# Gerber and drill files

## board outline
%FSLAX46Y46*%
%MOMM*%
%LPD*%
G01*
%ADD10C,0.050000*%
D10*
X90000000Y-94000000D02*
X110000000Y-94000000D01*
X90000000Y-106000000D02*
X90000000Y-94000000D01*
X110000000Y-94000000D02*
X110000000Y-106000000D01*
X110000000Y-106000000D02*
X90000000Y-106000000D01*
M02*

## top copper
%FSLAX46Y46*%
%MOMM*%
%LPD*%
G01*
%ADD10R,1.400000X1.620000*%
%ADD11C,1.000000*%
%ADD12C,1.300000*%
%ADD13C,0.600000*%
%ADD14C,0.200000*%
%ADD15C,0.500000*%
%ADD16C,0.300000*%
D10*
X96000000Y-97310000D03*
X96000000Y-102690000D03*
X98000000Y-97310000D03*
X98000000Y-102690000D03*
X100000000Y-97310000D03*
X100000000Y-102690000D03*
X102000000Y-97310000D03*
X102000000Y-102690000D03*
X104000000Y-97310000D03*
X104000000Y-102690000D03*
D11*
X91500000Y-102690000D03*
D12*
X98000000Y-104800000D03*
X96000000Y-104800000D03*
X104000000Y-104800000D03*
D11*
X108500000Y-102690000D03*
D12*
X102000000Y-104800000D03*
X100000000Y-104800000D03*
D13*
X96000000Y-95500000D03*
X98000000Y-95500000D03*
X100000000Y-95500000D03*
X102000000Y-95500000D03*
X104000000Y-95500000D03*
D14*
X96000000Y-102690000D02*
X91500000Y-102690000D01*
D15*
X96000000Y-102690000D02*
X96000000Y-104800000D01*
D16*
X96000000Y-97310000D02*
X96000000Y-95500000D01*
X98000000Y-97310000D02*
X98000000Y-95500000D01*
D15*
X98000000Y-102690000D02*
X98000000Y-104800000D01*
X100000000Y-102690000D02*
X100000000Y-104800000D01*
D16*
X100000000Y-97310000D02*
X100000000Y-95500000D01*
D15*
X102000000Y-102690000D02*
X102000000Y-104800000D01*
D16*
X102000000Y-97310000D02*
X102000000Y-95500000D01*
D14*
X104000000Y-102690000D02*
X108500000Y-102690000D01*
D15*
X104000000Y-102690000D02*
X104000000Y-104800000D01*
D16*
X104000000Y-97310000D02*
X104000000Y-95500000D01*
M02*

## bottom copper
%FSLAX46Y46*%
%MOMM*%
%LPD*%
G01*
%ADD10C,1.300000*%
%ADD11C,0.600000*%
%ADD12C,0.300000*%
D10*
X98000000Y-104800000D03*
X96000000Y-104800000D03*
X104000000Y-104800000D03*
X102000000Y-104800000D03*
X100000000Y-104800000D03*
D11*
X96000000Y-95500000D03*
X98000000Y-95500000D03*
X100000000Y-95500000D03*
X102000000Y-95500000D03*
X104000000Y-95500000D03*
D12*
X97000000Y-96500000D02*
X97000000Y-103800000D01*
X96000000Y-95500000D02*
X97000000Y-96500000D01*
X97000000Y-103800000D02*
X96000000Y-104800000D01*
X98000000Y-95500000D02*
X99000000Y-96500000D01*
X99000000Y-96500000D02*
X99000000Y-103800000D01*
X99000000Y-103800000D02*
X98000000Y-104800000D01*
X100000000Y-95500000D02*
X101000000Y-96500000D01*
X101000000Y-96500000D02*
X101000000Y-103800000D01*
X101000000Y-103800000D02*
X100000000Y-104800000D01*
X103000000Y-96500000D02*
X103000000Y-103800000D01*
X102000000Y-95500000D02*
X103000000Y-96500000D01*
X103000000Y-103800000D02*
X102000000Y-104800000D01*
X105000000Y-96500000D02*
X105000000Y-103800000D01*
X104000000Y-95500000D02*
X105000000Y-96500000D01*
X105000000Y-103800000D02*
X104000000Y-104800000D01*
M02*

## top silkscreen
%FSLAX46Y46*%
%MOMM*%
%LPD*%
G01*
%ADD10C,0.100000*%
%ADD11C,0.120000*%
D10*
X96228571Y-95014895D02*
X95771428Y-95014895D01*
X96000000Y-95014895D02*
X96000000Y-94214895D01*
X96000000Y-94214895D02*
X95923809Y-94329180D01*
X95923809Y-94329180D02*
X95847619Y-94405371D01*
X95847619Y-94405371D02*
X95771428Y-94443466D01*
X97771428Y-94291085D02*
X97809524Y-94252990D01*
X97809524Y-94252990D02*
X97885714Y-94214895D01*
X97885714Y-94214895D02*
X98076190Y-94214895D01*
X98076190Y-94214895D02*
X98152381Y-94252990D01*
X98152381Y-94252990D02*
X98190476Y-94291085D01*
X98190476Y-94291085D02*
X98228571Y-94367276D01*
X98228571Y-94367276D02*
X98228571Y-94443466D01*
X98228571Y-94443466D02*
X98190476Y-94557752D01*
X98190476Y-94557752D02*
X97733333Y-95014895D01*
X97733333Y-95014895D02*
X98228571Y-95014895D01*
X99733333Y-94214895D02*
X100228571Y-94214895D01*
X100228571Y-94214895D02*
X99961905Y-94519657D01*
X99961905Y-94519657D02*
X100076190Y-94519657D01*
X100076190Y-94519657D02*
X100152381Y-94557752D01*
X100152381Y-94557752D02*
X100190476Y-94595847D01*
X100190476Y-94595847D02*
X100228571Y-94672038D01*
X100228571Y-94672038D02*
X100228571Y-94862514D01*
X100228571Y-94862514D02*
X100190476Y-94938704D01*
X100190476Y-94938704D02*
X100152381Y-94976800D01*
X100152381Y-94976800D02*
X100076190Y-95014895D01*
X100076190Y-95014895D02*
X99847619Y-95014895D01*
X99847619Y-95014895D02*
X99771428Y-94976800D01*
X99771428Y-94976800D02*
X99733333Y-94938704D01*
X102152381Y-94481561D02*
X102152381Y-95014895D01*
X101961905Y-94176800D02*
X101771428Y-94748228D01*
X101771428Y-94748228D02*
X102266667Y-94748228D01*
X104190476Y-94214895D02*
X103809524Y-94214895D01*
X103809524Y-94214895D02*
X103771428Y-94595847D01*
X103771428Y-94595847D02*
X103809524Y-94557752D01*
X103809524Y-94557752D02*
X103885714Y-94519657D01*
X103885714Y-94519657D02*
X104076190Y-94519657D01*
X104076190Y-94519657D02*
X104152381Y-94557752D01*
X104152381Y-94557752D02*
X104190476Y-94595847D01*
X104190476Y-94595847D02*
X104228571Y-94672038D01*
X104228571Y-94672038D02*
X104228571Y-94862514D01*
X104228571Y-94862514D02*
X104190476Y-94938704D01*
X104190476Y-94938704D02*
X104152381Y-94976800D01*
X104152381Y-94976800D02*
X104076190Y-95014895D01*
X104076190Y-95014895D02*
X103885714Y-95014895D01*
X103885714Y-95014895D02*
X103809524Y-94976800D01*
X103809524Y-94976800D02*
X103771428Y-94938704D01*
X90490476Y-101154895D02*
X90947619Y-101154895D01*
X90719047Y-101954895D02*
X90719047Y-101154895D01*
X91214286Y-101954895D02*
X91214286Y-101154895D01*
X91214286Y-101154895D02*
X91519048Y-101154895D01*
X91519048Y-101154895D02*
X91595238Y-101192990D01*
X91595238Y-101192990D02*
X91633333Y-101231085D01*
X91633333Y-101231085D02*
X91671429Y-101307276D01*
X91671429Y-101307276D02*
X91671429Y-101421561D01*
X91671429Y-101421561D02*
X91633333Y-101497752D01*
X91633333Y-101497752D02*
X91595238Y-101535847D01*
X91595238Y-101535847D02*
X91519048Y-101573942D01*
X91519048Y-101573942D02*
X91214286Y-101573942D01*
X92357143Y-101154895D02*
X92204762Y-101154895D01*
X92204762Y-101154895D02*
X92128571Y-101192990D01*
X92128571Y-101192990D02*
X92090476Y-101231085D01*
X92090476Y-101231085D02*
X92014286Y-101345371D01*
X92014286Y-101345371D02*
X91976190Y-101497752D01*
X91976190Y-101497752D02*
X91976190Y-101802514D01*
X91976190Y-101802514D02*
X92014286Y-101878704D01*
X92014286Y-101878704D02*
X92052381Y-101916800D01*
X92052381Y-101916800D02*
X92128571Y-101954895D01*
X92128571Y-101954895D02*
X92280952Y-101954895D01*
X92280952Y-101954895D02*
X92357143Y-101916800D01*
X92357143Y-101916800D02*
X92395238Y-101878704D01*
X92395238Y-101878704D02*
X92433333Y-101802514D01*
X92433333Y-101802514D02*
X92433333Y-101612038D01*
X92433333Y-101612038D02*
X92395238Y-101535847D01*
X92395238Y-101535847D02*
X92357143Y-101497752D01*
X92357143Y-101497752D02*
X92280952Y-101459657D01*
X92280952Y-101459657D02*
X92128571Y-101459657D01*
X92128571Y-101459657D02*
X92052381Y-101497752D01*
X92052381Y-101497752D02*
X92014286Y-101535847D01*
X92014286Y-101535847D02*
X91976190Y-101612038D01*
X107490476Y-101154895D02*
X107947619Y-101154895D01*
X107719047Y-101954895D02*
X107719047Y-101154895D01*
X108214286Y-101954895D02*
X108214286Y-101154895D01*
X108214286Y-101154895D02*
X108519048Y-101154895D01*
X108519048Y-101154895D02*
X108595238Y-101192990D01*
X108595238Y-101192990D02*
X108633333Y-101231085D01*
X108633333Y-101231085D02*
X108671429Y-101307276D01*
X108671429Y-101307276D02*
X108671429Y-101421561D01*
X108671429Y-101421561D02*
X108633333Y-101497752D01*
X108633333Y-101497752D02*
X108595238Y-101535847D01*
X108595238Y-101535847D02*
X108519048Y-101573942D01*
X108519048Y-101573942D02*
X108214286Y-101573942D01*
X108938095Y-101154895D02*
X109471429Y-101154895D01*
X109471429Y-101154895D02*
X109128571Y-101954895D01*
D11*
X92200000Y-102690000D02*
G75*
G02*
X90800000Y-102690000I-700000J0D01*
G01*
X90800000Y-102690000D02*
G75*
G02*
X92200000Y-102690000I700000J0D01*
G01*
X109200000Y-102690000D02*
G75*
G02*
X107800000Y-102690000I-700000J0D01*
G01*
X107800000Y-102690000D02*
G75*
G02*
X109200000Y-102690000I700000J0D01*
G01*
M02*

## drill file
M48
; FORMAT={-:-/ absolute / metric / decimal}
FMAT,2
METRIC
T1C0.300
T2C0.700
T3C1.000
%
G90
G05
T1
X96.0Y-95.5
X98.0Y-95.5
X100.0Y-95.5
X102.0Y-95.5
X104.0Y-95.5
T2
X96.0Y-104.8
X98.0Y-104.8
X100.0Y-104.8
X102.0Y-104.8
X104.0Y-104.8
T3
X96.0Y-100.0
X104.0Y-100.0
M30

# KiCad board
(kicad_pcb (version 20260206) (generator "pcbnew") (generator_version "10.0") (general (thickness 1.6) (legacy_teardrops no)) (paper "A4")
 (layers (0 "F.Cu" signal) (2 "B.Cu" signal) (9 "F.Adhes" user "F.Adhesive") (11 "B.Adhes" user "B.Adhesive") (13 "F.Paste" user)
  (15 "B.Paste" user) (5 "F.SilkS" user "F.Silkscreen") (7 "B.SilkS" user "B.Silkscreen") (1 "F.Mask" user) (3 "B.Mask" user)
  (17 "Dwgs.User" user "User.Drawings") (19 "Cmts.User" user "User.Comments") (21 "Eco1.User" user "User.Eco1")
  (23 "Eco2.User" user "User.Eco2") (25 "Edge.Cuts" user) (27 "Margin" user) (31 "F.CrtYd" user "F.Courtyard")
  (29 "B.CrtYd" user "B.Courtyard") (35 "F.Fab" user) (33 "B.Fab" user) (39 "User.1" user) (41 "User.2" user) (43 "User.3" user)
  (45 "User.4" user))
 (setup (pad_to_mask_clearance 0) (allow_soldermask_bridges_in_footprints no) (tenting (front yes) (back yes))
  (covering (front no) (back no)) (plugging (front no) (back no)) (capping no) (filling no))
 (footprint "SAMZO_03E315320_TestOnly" (layer "F.Cu") (at 100 100)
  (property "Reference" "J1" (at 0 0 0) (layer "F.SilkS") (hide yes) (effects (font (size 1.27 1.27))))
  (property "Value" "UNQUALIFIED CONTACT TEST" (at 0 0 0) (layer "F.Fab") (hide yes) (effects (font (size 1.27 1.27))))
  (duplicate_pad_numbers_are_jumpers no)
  (pad "" np_thru_hole circle (at -4 0) (size 1 1) (drill 1) (layers "*.Cu"))
  (pad "" np_thru_hole circle (at 4 0) (size 1 1) (drill 1) (layers "*.Cu"))
  (pad "1" smd rect (at -4 -2.69) (size 1.4 1.62) (layers "F.Cu" "F.Mask" "F.Paste") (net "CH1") (thermal_bridge_angle 45))
  (pad "1" smd rect (at -4 2.69) (size 1.4 1.62) (layers "F.Cu" "F.Mask" "F.Paste") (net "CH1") (thermal_bridge_angle 45))
  (pad "2" smd rect (at -2 -2.69) (size 1.4 1.62) (layers "F.Cu" "F.Mask" "F.Paste") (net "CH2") (thermal_bridge_angle 45))
  (pad "2" smd rect (at -2 2.69) (size 1.4 1.62) (layers "F.Cu" "F.Mask" "F.Paste") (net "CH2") (thermal_bridge_angle 45))
  (pad "3" smd rect (at 0 -2.69) (size 1.4 1.62) (layers "F.Cu" "F.Mask" "F.Paste") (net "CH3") (thermal_bridge_angle 45))
  (pad "3" smd rect (at 0 2.69) (size 1.4 1.62) (layers "F.Cu" "F.Mask" "F.Paste") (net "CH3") (thermal_bridge_angle 45))
  (pad "4" smd rect (at 2 -2.69) (size 1.4 1.62) (layers "F.Cu" "F.Mask" "F.Paste") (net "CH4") (thermal_bridge_angle 45))
  (pad "4" smd rect (at 2 2.69) (size 1.4 1.62) (layers "F.Cu" "F.Mask" "F.Paste") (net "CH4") (thermal_bridge_angle 45))
  (pad "5" smd rect (at 4 -2.69) (size 1.4 1.62) (layers "F.Cu" "F.Mask" "F.Paste") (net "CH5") (thermal_bridge_angle 45))
  (pad "5" smd rect (at 4 2.69) (size 1.4 1.62) (layers "F.Cu" "F.Mask" "F.Paste") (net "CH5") (thermal_bridge_angle 45)))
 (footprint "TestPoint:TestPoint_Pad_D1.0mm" (layer "F.Cu") (at 91.5 102.69)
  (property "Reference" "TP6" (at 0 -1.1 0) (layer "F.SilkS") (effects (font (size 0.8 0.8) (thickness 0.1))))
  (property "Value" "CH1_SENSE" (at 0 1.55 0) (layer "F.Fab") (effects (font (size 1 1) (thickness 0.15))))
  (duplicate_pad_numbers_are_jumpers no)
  (fp_circle (center 0 0) (end 0 0.7) (stroke (width 0.12) (type solid)) (fill no) (layer "F.SilkS"))
  (pad "1" smd circle (at 0 0) (size 1 1) (layers "F.Cu" "F.Mask") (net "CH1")))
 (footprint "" (layer "F.Cu") (at 98 104.8)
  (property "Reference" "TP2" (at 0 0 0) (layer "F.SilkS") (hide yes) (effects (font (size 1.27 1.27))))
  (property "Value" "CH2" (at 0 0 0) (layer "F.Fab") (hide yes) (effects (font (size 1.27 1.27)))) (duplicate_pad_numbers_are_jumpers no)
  (pad "1" thru_hole circle (at 0 0) (size 1.3 1.3) (drill 0.7) (layers "*.Cu") (remove_unused_layers no) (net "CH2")))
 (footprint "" (layer "F.Cu") (at 96 104.8)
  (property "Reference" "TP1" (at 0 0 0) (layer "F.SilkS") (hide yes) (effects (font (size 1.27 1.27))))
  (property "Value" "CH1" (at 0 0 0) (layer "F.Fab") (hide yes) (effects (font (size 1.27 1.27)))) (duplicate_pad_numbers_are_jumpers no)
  (pad "1" thru_hole circle (at 0 0) (size 1.3 1.3) (drill 0.7) (layers "*.Cu") (remove_unused_layers no) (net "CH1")))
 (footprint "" (layer "F.Cu") (at 104 104.8)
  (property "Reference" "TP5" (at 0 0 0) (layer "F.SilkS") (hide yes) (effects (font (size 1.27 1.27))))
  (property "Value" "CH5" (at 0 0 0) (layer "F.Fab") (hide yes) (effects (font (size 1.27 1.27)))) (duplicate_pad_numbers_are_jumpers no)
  (pad "1" thru_hole circle (at 0 0) (size 1.3 1.3) (drill 0.7) (layers "*.Cu") (remove_unused_layers no) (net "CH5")))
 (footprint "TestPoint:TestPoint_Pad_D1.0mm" (layer "F.Cu") (at 108.5 102.69)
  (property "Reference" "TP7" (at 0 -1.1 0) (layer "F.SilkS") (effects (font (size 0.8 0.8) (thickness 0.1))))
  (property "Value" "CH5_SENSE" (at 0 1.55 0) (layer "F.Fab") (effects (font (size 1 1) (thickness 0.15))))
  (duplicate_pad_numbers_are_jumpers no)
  (fp_circle (center 0 0) (end 0 0.7) (stroke (width 0.12) (type solid)) (fill no) (layer "F.SilkS"))
  (pad "1" smd circle (at 0 0) (size 1 1) (layers "F.Cu" "F.Mask") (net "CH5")))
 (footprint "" (layer "F.Cu") (at 102 104.8)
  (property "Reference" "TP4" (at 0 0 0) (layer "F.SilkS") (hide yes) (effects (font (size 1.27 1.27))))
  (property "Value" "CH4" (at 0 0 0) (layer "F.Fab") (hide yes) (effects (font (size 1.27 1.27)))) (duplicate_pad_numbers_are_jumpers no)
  (pad "1" thru_hole circle (at 0 0) (size 1.3 1.3) (drill 0.7) (layers "*.Cu") (remove_unused_layers no) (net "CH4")))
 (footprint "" (layer "F.Cu") (at 100 104.8)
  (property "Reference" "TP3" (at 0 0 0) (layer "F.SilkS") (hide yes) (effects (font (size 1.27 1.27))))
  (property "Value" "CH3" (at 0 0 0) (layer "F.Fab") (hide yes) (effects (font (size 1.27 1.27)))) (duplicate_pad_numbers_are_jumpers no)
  (pad "1" thru_hole circle (at 0 0) (size 1.3 1.3) (drill 0.7) (layers "*.Cu") (remove_unused_layers no) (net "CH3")))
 (gr_line (start 90 94) (end 110 94) (stroke (width 0.05) (type default)) (layer "Edge.Cuts"))
 (gr_line (start 90 106) (end 90 94) (stroke (width 0.05) (type default)) (layer "Edge.Cuts"))
 (gr_line (start 110 94) (end 110 106) (stroke (width 0.05) (type default)) (layer "Edge.Cuts"))
 (gr_line (start 110 106) (end 90 106) (stroke (width 0.05) (type default)) (layer "Edge.Cuts"))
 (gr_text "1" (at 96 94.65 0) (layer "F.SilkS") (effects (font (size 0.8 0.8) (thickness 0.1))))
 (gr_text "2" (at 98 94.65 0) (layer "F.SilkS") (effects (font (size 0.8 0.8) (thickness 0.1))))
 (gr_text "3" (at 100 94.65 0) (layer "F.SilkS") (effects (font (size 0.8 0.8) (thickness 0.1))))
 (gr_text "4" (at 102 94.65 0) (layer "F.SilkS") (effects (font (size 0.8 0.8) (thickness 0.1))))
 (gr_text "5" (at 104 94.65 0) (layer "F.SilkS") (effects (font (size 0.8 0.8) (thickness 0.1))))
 (segment (start 96 102.69) (end 91.5 102.69) (width 0.2) (layer "F.Cu") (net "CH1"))
 (segment (start 96 102.69) (end 96 104.8) (width 0.5) (layer "F.Cu") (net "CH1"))
 (segment (start 96 97.31) (end 96 95.5) (width 0.3) (layer "F.Cu") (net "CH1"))
 (via (at 96 95.5) (size 0.6) (drill 0.3) (layers "F.Cu" "B.Cu") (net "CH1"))
 (segment (start 97 96.5) (end 97 103.8) (width 0.3) (layer "B.Cu") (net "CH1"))
 (segment (start 96 95.5) (end 97 96.5) (width 0.3) (layer "B.Cu") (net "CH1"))
 (segment (start 97 103.8) (end 96 104.8) (width 0.3) (layer "B.Cu") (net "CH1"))
 (segment (start 98 97.31) (end 98 95.5) (width 0.3) (layer "F.Cu") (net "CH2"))
 (segment (start 98 102.69) (end 98 104.8) (width 0.5) (layer "F.Cu") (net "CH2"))
 (via (at 98 95.5) (size 0.6) (drill 0.3) (layers "F.Cu" "B.Cu") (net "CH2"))
 (segment (start 98 95.5) (end 99 96.5) (width 0.3) (layer "B.Cu") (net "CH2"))
 (segment (start 99 96.5) (end 99 103.8) (width 0.3) (layer "B.Cu") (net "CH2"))
 (segment (start 99 103.8) (end 98 104.8) (width 0.3) (layer "B.Cu") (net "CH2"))
 (segment (start 100 102.69) (end 100 104.8) (width 0.5) (layer "F.Cu") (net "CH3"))
 (segment (start 100 97.31) (end 100 95.5) (width 0.3) (layer "F.Cu") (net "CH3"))
 (via (at 100 95.5) (size 0.6) (drill 0.3) (layers "F.Cu" "B.Cu") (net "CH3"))
 (segment (start 100 95.5) (end 101 96.5) (width 0.3) (layer "B.Cu") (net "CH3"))
 (segment (start 101 96.5) (end 101 103.8) (width 0.3) (layer "B.Cu") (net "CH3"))
 (segment (start 101 103.8) (end 100 104.8) (width 0.3) (layer "B.Cu") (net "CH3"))
 (segment (start 102 102.69) (end 102 104.8) (width 0.5) (layer "F.Cu") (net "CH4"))
 (segment (start 102 97.31) (end 102 95.5) (width 0.3) (layer "F.Cu") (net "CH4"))
 (via (at 102 95.5) (size 0.6) (drill 0.3) (layers "F.Cu" "B.Cu") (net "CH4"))
 (segment (start 103 96.5) (end 103 103.8) (width 0.3) (layer "B.Cu") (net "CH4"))
 (segment (start 102 95.5) (end 103 96.5) (width 0.3) (layer "B.Cu") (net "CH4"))
 (segment (start 103 103.8) (end 102 104.8) (width 0.3) (layer "B.Cu") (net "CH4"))
 (segment (start 104 102.69) (end 108.5 102.69) (width 0.2) (layer "F.Cu") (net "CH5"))
 (segment (start 104 102.69) (end 104 104.8) (width 0.5) (layer "F.Cu") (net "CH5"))
 (segment (start 104 97.31) (end 104 95.5) (width 0.3) (layer "F.Cu") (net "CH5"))
 (via (at 104 95.5) (size 0.6) (drill 0.3) (layers "F.Cu" "B.Cu") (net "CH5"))
 (segment (start 105 96.5) (end 105 103.8) (width 0.3) (layer "B.Cu") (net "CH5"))
 (segment (start 104 95.5) (end 105 96.5) (width 0.3) (layer "B.Cu") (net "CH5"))
 (segment (start 105 103.8) (end 104 104.8) (width 0.3) (layer "B.Cu") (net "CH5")))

